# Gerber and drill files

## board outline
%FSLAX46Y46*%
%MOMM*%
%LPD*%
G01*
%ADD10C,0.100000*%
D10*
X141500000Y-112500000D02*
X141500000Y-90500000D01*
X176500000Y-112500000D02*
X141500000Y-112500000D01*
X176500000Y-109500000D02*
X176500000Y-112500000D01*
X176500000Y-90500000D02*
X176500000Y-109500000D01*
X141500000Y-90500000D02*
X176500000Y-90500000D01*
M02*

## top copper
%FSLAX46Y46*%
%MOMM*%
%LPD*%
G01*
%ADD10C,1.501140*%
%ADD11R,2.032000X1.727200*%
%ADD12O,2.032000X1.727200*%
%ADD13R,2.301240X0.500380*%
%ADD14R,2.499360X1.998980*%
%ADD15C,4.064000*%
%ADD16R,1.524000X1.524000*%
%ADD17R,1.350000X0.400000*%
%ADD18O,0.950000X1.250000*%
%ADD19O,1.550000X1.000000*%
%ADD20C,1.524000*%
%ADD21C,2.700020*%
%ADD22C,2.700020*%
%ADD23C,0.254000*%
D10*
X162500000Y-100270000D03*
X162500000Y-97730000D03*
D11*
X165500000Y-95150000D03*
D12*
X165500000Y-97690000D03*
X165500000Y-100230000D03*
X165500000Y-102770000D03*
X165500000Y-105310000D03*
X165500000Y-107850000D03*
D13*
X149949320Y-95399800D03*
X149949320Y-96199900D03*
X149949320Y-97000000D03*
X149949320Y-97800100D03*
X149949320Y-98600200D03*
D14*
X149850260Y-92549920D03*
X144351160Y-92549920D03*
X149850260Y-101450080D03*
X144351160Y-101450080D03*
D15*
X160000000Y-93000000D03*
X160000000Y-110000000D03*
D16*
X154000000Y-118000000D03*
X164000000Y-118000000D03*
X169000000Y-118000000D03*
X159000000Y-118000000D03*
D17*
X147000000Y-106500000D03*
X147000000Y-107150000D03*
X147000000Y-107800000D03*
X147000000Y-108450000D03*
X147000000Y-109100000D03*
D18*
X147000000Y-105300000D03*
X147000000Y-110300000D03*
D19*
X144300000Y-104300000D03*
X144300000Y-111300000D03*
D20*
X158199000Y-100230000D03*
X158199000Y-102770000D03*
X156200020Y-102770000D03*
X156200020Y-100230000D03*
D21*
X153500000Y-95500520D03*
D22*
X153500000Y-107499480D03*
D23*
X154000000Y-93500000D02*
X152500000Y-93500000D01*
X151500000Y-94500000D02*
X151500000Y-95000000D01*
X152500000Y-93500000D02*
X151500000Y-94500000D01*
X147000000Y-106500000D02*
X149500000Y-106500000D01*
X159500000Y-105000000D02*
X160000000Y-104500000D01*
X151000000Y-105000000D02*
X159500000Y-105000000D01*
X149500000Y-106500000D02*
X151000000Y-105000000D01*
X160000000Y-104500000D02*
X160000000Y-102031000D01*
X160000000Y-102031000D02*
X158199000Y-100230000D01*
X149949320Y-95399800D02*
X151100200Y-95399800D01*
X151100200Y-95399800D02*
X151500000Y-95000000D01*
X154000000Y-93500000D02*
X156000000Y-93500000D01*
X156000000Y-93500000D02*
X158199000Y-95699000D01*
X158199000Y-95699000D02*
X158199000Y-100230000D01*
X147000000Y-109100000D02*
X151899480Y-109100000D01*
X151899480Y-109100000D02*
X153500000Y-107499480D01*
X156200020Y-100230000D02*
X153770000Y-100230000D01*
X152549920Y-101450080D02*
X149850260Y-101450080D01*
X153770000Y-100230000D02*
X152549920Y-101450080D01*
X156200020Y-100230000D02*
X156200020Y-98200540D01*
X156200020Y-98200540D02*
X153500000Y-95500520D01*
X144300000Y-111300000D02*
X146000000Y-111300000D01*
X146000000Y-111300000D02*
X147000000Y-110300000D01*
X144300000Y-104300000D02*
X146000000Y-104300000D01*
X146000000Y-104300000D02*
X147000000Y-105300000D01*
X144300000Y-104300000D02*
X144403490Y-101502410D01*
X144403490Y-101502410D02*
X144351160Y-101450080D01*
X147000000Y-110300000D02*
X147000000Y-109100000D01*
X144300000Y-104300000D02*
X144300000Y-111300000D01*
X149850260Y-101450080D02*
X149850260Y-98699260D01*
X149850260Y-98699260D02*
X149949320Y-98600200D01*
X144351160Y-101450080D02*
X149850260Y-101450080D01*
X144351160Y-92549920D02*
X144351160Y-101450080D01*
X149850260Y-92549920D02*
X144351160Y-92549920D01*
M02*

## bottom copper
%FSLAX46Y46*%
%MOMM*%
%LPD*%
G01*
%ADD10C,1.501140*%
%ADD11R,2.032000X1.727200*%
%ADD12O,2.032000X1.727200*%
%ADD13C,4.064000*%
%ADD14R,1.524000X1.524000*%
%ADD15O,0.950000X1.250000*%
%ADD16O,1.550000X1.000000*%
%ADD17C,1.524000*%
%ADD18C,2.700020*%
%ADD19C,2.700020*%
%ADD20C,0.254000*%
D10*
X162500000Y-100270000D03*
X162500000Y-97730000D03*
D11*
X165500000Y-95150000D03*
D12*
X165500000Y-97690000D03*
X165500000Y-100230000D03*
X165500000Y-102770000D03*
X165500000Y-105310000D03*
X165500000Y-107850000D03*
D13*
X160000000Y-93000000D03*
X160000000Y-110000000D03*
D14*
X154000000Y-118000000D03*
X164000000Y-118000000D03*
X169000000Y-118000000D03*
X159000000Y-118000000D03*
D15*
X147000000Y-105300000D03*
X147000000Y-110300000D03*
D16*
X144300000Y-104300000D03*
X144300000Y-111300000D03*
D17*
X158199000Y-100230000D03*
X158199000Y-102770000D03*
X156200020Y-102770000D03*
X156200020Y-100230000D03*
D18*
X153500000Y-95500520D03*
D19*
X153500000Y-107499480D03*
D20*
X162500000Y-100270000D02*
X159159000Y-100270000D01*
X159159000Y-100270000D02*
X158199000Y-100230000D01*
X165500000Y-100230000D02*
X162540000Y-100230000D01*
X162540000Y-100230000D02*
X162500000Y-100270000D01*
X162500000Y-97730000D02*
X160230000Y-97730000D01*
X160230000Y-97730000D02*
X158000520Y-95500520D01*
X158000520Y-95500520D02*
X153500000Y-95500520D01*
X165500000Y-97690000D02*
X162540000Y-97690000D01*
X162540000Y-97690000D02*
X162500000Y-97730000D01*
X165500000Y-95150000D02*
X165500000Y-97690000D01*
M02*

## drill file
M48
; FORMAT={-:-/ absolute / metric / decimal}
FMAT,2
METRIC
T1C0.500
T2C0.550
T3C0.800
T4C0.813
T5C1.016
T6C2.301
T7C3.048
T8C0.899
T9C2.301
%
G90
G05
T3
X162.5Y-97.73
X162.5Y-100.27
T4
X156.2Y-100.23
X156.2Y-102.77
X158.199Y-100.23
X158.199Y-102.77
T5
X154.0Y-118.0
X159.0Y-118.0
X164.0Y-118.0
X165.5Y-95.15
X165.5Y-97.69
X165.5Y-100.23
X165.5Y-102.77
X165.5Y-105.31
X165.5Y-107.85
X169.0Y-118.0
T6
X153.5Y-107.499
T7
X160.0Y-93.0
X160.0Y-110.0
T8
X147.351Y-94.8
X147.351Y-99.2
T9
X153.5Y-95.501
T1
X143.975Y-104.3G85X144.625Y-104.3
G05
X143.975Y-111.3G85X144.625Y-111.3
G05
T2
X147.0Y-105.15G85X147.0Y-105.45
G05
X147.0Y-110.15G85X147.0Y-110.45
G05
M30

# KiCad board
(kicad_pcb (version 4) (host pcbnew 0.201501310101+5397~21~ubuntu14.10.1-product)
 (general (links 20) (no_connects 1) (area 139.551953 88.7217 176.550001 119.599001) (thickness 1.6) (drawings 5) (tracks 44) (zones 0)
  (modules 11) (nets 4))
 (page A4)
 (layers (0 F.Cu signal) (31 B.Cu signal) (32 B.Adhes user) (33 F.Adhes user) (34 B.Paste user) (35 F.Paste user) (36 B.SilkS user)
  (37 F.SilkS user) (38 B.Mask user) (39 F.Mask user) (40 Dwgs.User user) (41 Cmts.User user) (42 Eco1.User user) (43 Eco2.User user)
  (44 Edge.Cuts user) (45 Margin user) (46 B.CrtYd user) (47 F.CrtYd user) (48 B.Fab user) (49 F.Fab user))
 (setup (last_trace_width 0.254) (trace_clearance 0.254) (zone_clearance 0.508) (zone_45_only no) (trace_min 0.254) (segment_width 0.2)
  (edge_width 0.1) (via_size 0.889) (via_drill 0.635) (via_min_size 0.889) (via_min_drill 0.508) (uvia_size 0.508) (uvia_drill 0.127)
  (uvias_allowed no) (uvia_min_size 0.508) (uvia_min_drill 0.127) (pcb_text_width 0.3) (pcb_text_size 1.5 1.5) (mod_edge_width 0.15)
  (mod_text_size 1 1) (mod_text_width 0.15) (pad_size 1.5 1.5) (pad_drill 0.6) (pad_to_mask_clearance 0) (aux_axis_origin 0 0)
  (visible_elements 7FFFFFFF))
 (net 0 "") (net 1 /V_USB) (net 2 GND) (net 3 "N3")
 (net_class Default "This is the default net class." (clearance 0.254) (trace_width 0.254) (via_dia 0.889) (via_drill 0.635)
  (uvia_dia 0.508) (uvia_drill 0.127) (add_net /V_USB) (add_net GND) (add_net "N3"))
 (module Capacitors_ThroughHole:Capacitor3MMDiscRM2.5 (layer F.Cu) (at 162.5 99 90)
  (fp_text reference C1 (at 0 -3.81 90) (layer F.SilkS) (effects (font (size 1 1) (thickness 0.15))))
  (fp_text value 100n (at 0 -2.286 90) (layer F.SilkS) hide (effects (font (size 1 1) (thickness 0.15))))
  (pad 1 thru_hole circle (at -1.27 0 90) (size 1.50114 1.50114) (drill 0.8001) (layers *.Cu *.Mask F.SilkS) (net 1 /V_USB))
  (pad 2 thru_hole circle (at 1.27 0 90) (size 1.50114 1.50114) (drill 0.8001) (layers *.Cu *.Mask F.SilkS) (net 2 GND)))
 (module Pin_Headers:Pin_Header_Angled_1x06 (layer F.Cu) (at 165.5 101.5 270)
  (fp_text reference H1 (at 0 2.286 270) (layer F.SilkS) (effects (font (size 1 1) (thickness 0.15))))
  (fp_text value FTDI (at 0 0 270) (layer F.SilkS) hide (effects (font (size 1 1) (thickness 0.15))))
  (pad 1 thru_hole rect (at -6.35 0 270) (size 1.7272 2.032) (drill 1.016) (layers *.Cu *.Mask F.SilkS) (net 2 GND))
  (pad 2 thru_hole oval (at -3.81 0 270) (size 1.7272 2.032) (drill 1.016) (layers *.Cu *.Mask F.SilkS) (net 2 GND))
  (pad 3 thru_hole oval (at -1.27 0 270) (size 1.7272 2.032) (drill 1.016) (layers *.Cu *.Mask F.SilkS) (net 1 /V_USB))
  (pad 4 thru_hole oval (at 1.27 0 270) (size 1.7272 2.032) (drill 1.016) (layers *.Cu *.Mask F.SilkS))
  (pad 5 thru_hole oval (at 3.81 0 270) (size 1.7272 2.032) (drill 1.016) (layers *.Cu *.Mask F.SilkS))
  (pad 6 thru_hole oval (at 6.35 0 270) (size 1.7272 2.032) (drill 1.016) (layers *.Cu *.Mask F.SilkS)))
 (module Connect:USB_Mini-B (layer F.Cu) (at 146.5 97)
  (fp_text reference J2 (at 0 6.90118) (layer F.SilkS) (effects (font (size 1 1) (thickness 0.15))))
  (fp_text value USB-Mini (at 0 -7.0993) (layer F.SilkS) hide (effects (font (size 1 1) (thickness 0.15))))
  (pad 1 smd rect (at 3.44932 -1.6002) (size 2.30124 0.50038) (layers F.Cu F.Paste F.Mask) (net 1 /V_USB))
  (pad 2 smd rect (at 3.44932 -0.8001) (size 2.30124 0.50038) (layers F.Cu F.Paste F.Mask) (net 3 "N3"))
  (pad 3 smd rect (at 3.44932 0) (size 2.30124 0.50038) (layers F.Cu F.Paste F.Mask))
  (pad 4 smd rect (at 3.44932 0.8001) (size 2.30124 0.50038) (layers F.Cu F.Paste F.Mask))
  (pad 5 smd rect (at 3.44932 1.6002) (size 2.30124 0.50038) (layers F.Cu F.Paste F.Mask) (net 2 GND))
  (pad 6 smd rect (at 3.35026 -4.45008) (size 2.49936 1.99898) (layers F.Cu F.Paste F.Mask) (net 2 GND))
  (pad 7 smd rect (at -2.14884 -4.45008) (size 2.49936 1.99898) (layers F.Cu F.Paste F.Mask) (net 2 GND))
  (pad 8 smd rect (at 3.35026 4.45008) (size 2.49936 1.99898) (layers F.Cu F.Paste F.Mask) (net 2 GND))
  (pad 9 smd rect (at -2.14884 4.45008) (size 2.49936 1.99898) (layers F.Cu F.Paste F.Mask) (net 2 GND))
  (pad "" np_thru_hole circle (at 0.8509 -2.19964) (size 0.89916 0.89916) (drill 0.89916) (layers *.Cu *.Mask F.SilkS))
  (pad 2 np_thru_hole circle (at 0.8509 2.19964) (size 0.89916 0.89916) (drill 0.89916) (layers *.Cu *.Mask F.SilkS) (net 3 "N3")))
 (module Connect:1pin (layer F.Cu) (at 160 93)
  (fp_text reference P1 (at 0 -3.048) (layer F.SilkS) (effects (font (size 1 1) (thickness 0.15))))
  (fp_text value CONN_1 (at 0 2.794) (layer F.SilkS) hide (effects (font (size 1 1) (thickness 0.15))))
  (pad 1 thru_hole circle (at 0 0) (size 4.064 4.064) (drill 3.048) (layers *.Cu *.Mask F.SilkS)))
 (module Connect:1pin (layer F.Cu) (at 160 110)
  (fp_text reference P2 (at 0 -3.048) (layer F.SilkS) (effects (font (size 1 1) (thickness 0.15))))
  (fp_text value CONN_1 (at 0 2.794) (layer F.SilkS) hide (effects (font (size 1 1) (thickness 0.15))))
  (pad 1 thru_hole circle (at 0 0) (size 4.064 4.064) (drill 3.048) (layers *.Cu *.Mask F.SilkS)))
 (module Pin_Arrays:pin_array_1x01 (layer F.Cu) (at 154 118)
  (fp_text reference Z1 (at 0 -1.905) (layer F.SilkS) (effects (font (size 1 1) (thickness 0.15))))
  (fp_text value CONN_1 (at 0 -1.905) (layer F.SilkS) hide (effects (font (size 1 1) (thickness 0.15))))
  (pad 1 thru_hole rect (at 0 0) (size 1.524 1.524) (drill 1.016) (layers *.Cu *.Mask F.SilkS)))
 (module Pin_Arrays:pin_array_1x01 (layer F.Cu) (at 164 118)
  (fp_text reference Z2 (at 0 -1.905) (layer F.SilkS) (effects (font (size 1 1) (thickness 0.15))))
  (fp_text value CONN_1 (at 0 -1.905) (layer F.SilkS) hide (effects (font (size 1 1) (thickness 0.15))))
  (pad 1 thru_hole rect (at 0 0) (size 1.524 1.524) (drill 1.016) (layers *.Cu *.Mask F.SilkS)))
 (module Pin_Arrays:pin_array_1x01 (layer F.Cu) (at 169 118)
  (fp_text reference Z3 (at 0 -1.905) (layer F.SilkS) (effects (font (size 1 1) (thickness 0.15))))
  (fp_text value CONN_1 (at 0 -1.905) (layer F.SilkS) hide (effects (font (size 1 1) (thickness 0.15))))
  (pad 1 thru_hole rect (at 0 0) (size 1.524 1.524) (drill 1.016) (layers *.Cu *.Mask F.SilkS)))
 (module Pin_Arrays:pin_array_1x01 (layer F.Cu) (at 159 118)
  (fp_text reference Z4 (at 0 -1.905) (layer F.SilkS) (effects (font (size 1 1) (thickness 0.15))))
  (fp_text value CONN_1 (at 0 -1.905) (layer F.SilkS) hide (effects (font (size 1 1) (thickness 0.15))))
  (pad 1 thru_hole rect (at 0 0) (size 1.524 1.524) (drill 1.016) (layers *.Cu *.Mask F.SilkS)))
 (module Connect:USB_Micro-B (layer F.Cu) (at 147 106.5)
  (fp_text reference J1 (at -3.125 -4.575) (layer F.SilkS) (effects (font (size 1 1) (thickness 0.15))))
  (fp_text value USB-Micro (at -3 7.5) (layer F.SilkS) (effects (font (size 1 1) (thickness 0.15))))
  (pad 1 smd rect (at 0 0) (size 1.35 0.4) (layers F.Cu F.Paste F.Mask) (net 1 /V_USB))
  (pad 2 smd rect (at 0 0.65) (size 1.35 0.4) (layers F.Cu F.Paste F.Mask))
  (pad 3 smd rect (at 0 1.3) (size 1.35 0.4) (layers F.Cu F.Paste F.Mask))
  (pad 4 smd rect (at 0 1.95) (size 1.35 0.4) (layers F.Cu F.Paste F.Mask))
  (pad 5 smd rect (at 0 2.6) (size 1.35 0.4) (layers F.Cu F.Paste F.Mask) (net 2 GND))
  (pad 6 thru_hole oval (at 0 -1.2) (size 0.95 1.25) (drill oval 0.55 0.85) (layers *.Cu *.Mask F.SilkS) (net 2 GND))
  (pad 7 thru_hole oval (at 0 3.8) (size 0.95 1.25) (drill oval 0.55 0.85) (layers *.Cu *.Mask F.SilkS) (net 2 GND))
  (pad 8 thru_hole oval (at -2.7 -2.2) (size 1.55 1) (drill oval 1.15 0.5) (layers *.Cu *.Mask F.SilkS) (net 2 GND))
  (pad 9 thru_hole oval (at -2.7 4.8) (size 1.55 1) (drill oval 1.15 0.5) (layers *.Cu *.Mask F.SilkS) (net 2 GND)))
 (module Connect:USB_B (layer B.Cu) (at 153.5 101.5 90)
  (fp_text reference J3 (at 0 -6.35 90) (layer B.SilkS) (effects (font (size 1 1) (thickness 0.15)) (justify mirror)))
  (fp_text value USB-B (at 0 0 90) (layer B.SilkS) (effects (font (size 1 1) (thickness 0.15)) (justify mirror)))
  (pad 1 thru_hole circle (at 1.27 4.699 90) (size 1.524 1.524) (drill 0.8128) (layers *.Cu *.Mask B.SilkS) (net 1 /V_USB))
  (pad 2 thru_hole circle (at -1.27 4.699 90) (size 1.524 1.524) (drill 0.8128) (layers *.Cu *.Mask B.SilkS))
  (pad 3 thru_hole circle (at -1.27 2.70002 90) (size 1.524 1.524) (drill 0.8128) (layers *.Cu *.Mask B.SilkS))
  (pad 4 thru_hole circle (at 1.27 2.70002 90) (size 1.524 1.524) (drill 0.8128) (layers *.Cu *.Mask B.SilkS) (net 2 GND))
  (pad 5 np_thru_hole circle (at 5.99948 0 90) (size 2.70002 2.70002) (drill 2.30124) (layers *.Cu *.SilkS *.Mask) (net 2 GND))
  (pad 6 thru_hole circle (at -5.99948 0 90) (size 2.70002 2.70002) (drill 2.30124) (layers *.Cu *.Mask B.SilkS) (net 2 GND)))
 (gr_line (start 141.5 112.5) (end 141.5 90.5) (angle 90) (layer Edge.Cuts) (width 0.1))
 (gr_line (start 176.5 112.5) (end 141.5 112.5) (angle 90) (layer Edge.Cuts) (width 0.1))
 (gr_line (start 176.5 109.5) (end 176.5 112.5) (angle 90) (layer Edge.Cuts) (width 0.1))
 (gr_line (start 176.5 90.5) (end 176.5 109.5) (angle 90) (layer Edge.Cuts) (width 0.1))
 (gr_line (start 141.5 90.5) (end 176.5 90.5) (angle 90) (layer Edge.Cuts) (width 0.1))
 (segment (start 154 93.5) (end 152.5 93.5) (width 0.254) (layer F.Cu) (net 1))
 (segment (start 151.5 94.5) (end 151.5 95) (width 0.254) (layer F.Cu) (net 1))
 (segment (start 152.5 93.5) (end 151.5 94.5) (width 0.254) (layer F.Cu) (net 1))
 (segment (start 147 106.5) (end 149.5 106.5) (width 0.254) (layer F.Cu) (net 1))
 (segment (start 159.5 105) (end 160 104.5) (width 0.254) (layer F.Cu) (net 1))
 (segment (start 151 105) (end 159.5 105) (width 0.254) (layer F.Cu) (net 1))
 (segment (start 149.5 106.5) (end 151 105) (width 0.254) (layer F.Cu) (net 1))
 (segment (start 160 104.5) (end 160 102.031) (width 0.254) (layer F.Cu) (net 1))
 (segment (start 160 102.031) (end 158.199 100.23) (width 0.254) (layer F.Cu) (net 1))
 (segment (start 162.5 100.27) (end 159.159 100.27) (width 0.254) (layer B.Cu) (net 1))
 (segment (start 159.159 100.27) (end 158.199 100.23) (width 0.254) (layer B.Cu) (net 1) (status 20))
 (segment (start 149.94932 95.3998) (end 151.1002 95.3998) (width 0.254) (layer F.Cu) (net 1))
 (segment (start 151.1002 95.3998) (end 151.5 95) (width 0.254) (layer F.Cu) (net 1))
 (segment (start 154 93.5) (end 156 93.5) (width 0.254) (layer F.Cu) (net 1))
 (segment (start 156 93.5) (end 158.199 95.699) (width 0.254) (layer F.Cu) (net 1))
 (segment (start 158.199 95.699) (end 158.199 100.23) (width 0.254) (layer F.Cu) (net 1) (status 20))
 (segment (start 165.5 100.23) (end 162.54 100.23) (width 0.254) (layer B.Cu) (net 1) (status 20))
 (segment (start 162.54 100.23) (end 162.5 100.27) (width 0.254) (layer B.Cu) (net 1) (status 30))
 (segment (start 147 109.1) (end 151.89948 109.1) (width 0.254) (layer F.Cu) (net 2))
 (segment (start 151.89948 109.1) (end 153.5 107.49948) (width 0.254) (layer F.Cu) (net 2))
 (segment (start 156.20002 100.23) (end 153.77 100.23) (width 0.254) (layer F.Cu) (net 2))
 (segment (start 152.54992 101.45008) (end 149.85026 101.45008) (width 0.254) (layer F.Cu) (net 2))
 (segment (start 153.77 100.23) (end 152.54992 101.45008) (width 0.254) (layer F.Cu) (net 2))
 (segment (start 156.20002 100.23) (end 156.20002 98.20054) (width 0.254) (layer F.Cu) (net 2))
 (segment (start 156.20002 98.20054) (end 153.5 95.50052) (width 0.254) (layer F.Cu) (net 2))
 (segment (start 162.5 97.73) (end 160.23 97.73) (width 0.254) (layer B.Cu) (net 2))
 (segment (start 160.23 97.73) (end 158.00052 95.50052) (width 0.254) (layer B.Cu) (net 2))
 (segment (start 158.00052 95.50052) (end 153.5 95.50052) (width 0.254) (layer B.Cu) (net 2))
 (segment (start 144.3 111.3) (end 146 111.3) (width 0.254) (layer F.Cu) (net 2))
 (segment (start 146 111.3) (end 147 110.3) (width 0.254) (layer F.Cu) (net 2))
 (segment (start 144.3 104.3) (end 146 104.3) (width 0.254) (layer F.Cu) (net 2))
 (segment (start 146 104.3) (end 147 105.3) (width 0.254) (layer F.Cu) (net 2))
 (segment (start 144.3 104.3) (end 144.40349 101.50241) (width 0.254) (layer F.Cu) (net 2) (status 10))
 (segment (start 144.40349 101.50241) (end 144.35116 101.45008) (width 0.254) (layer F.Cu) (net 2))
 (segment (start 147 110.3) (end 147 109.1) (width 0.254) (layer F.Cu) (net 2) (status 30))
 (segment (start 144.3 104.3) (end 144.3 111.3) (width 0.254) (layer F.Cu) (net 2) (status 30))
 (segment (start 149.85026 101.45008) (end 149.85026 98.69926) (width 0.254) (layer F.Cu) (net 2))
 (segment (start 149.85026 98.69926) (end 149.94932 98.6002) (width 0.254) (layer F.Cu) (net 2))
 (segment (start 144.35116 101.45008) (end 149.85026 101.45008) (width 0.254) (layer F.Cu) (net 2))
 (segment (start 144.35116 92.54992) (end 144.35116 101.45008) (width 0.254) (layer F.Cu) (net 2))
 (segment (start 149.85026 92.54992) (end 144.35116 92.54992) (width 0.254) (layer F.Cu) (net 2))
 (segment (start 165.5 97.69) (end 162.54 97.69) (width 0.254) (layer B.Cu) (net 2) (status 20))
 (segment (start 162.54 97.69) (end 162.5 97.73) (width 0.254) (layer B.Cu) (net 2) (status 30))
 (segment (start 165.5 95.15) (end 165.5 97.69) (width 0.254) (layer B.Cu) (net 2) (status 30)))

